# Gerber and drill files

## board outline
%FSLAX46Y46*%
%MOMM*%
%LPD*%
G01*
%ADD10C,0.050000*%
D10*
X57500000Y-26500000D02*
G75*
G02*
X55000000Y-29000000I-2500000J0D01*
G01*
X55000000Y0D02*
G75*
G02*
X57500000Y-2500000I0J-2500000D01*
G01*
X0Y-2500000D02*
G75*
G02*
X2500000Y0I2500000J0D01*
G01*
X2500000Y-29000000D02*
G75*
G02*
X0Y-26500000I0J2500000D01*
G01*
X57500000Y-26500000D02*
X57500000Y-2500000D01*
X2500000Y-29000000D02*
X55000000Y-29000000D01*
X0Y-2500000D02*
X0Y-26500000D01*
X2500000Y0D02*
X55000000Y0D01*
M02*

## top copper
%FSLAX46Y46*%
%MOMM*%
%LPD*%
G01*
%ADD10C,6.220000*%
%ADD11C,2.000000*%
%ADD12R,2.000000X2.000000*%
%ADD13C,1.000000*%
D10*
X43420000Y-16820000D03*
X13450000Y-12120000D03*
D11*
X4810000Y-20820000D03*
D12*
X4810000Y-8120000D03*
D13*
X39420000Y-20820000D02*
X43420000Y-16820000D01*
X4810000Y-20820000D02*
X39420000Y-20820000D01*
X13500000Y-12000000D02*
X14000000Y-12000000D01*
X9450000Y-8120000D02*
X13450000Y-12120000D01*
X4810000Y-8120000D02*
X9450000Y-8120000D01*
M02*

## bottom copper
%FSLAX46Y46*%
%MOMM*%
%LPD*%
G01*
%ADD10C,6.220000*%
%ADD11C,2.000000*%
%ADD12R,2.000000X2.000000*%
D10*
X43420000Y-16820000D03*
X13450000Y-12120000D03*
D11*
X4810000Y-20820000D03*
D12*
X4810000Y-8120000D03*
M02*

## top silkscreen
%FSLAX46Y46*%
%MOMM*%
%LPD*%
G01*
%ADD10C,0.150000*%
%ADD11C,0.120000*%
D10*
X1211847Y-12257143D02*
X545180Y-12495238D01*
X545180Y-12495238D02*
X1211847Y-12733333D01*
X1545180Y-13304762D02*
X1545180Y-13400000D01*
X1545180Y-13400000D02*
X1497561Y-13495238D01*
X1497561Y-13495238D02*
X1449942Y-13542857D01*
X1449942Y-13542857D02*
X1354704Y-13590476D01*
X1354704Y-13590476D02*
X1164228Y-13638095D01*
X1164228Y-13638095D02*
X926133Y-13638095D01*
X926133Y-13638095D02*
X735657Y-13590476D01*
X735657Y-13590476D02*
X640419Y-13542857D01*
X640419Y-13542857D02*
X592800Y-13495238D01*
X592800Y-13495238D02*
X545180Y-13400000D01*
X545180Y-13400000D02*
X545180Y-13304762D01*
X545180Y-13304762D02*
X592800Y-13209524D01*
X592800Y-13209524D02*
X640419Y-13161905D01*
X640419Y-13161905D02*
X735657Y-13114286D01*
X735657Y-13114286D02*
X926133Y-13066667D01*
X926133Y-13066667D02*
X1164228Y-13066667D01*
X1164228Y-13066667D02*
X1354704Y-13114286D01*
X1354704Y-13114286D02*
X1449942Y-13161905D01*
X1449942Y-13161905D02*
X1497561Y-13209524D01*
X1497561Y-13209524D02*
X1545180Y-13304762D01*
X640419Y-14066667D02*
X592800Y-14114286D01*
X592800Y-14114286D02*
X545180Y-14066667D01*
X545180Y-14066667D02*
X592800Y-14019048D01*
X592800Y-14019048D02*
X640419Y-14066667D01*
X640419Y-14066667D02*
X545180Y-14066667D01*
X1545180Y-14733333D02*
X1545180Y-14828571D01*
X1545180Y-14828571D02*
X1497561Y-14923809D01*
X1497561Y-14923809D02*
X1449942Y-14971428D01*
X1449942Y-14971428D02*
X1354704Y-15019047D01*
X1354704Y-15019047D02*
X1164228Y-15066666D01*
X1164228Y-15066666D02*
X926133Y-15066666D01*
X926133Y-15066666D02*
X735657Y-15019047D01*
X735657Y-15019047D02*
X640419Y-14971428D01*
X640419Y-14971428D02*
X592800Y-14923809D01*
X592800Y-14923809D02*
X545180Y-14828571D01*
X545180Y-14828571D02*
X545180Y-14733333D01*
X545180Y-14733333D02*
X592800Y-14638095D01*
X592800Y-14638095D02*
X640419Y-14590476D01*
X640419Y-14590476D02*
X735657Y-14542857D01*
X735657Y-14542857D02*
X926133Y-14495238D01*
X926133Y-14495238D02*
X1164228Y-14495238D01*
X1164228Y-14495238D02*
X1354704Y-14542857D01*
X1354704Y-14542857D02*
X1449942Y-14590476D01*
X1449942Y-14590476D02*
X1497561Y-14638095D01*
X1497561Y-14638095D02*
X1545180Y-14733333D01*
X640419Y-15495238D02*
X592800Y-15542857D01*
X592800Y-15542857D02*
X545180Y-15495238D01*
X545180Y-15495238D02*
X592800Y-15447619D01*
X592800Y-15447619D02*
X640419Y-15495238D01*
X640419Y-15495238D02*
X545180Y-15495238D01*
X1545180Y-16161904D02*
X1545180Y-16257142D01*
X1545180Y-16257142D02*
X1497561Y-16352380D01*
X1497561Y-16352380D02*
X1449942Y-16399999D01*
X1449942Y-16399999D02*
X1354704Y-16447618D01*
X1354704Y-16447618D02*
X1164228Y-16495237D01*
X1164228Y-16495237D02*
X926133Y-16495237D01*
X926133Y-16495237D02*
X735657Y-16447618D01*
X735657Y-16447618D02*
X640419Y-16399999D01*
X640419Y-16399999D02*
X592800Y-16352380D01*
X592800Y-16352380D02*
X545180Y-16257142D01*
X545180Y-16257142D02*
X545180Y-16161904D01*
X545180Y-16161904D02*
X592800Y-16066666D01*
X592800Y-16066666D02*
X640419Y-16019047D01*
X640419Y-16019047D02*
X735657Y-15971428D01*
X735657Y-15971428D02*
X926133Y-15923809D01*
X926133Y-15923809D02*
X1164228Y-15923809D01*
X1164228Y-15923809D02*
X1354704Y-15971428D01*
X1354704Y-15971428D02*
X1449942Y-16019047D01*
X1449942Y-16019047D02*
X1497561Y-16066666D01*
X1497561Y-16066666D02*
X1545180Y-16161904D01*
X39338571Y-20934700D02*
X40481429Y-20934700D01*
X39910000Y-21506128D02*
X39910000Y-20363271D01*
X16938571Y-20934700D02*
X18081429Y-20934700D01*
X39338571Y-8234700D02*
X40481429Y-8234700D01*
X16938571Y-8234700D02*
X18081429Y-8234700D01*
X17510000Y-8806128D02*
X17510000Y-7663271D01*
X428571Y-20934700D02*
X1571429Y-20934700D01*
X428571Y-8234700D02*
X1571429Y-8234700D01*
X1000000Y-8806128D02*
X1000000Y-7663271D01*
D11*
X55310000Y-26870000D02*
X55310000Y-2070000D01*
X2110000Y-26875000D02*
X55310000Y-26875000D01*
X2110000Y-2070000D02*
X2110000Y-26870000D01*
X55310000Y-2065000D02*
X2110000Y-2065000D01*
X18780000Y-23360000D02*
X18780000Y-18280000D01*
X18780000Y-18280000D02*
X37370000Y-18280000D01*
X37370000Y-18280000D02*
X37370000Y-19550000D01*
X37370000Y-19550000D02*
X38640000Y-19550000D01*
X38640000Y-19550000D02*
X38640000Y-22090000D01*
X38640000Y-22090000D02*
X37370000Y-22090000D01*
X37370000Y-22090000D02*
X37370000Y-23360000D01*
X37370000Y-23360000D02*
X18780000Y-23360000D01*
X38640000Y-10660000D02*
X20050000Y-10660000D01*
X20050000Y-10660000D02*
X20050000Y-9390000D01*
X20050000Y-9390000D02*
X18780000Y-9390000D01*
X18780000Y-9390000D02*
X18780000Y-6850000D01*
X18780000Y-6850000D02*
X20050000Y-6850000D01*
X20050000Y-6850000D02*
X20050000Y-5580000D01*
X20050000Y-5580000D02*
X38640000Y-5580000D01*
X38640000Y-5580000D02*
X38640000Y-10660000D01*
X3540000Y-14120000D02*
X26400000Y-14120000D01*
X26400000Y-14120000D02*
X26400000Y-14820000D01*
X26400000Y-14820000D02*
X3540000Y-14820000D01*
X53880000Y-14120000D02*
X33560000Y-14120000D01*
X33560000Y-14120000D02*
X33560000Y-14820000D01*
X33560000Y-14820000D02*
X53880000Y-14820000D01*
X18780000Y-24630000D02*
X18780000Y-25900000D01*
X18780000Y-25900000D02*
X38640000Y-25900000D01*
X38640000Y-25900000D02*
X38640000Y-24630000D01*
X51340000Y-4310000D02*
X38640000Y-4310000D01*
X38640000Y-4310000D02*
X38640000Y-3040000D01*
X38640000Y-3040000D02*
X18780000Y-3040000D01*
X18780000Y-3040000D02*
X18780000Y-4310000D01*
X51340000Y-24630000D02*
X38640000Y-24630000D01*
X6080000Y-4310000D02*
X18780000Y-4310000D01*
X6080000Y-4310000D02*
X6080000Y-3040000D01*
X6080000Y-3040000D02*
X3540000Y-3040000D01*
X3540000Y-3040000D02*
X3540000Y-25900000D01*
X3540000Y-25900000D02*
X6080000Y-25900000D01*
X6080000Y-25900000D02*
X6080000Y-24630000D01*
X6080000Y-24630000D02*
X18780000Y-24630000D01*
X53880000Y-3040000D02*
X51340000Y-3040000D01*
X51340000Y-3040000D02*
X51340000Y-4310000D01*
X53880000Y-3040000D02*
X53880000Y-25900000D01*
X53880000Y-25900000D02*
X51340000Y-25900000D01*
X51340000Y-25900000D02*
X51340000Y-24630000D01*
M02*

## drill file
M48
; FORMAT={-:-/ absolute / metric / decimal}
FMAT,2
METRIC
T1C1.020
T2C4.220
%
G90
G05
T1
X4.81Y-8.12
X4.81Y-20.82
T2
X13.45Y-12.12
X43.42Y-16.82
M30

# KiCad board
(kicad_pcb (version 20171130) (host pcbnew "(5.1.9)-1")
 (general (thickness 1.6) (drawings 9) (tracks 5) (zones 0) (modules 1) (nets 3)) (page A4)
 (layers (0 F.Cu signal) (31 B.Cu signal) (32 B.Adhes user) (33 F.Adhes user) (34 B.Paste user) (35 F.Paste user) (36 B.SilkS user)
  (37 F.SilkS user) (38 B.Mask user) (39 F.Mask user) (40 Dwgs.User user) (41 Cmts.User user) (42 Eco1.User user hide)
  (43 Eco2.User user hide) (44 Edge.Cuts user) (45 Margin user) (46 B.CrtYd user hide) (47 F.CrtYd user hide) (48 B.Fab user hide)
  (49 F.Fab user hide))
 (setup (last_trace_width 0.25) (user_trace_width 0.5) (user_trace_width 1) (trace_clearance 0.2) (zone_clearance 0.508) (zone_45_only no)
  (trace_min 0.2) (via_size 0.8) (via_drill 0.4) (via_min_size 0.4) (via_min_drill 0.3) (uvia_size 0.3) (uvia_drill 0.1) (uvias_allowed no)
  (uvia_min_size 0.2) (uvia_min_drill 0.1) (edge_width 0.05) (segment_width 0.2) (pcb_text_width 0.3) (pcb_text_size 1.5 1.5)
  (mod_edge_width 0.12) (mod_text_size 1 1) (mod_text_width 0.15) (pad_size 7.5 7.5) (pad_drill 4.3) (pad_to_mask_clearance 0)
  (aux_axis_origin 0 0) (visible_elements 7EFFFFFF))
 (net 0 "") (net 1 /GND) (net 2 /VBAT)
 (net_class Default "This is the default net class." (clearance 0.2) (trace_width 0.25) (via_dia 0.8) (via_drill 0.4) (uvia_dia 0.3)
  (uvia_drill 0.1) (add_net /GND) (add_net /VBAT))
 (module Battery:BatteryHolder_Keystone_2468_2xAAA (layer F.Cu) (at 4.81 8.12)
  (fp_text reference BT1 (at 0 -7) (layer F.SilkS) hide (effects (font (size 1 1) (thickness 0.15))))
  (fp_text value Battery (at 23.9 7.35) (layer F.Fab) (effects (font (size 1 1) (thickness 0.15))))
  (fp_line (start 50.5 18.75) (end 50.5 -6.05) (layer F.SilkS) (width 0.12))
  (fp_line (start -2.7 18.755) (end 50.5 18.755) (layer F.SilkS) (width 0.12))
  (fp_line (start -2.7 -6.05) (end -2.7 18.75) (layer F.SilkS) (width 0.12))
  (fp_line (start 50.5 -6.055) (end -2.7 -6.055) (layer F.SilkS) (width 0.12))
  (fp_line (start 13.97 15.24) (end 13.97 10.16) (layer F.SilkS) (width 0.12))
  (fp_line (start 13.97 10.16) (end 32.56 10.16) (layer F.SilkS) (width 0.12))
  (fp_line (start 32.56 10.16) (end 32.56 11.43) (layer F.SilkS) (width 0.12))
  (fp_line (start 32.56 11.43) (end 33.83 11.43) (layer F.SilkS) (width 0.12))
  (fp_line (start 33.83 11.43) (end 33.83 13.97) (layer F.SilkS) (width 0.12))
  (fp_line (start 33.83 13.97) (end 32.56 13.97) (layer F.SilkS) (width 0.12))
  (fp_line (start 32.56 13.97) (end 32.56 15.24) (layer F.SilkS) (width 0.12))
  (fp_line (start 32.56 15.24) (end 13.97 15.24) (layer F.SilkS) (width 0.12))
  (fp_line (start 33.83 2.54) (end 15.24 2.54) (layer F.SilkS) (width 0.12))
  (fp_line (start 15.24 2.54) (end 15.24 1.27) (layer F.SilkS) (width 0.12))
  (fp_line (start 15.24 1.27) (end 13.97 1.27) (layer F.SilkS) (width 0.12))
  (fp_line (start 13.97 1.27) (end 13.97 -1.27) (layer F.SilkS) (width 0.12))
  (fp_line (start 13.97 -1.27) (end 15.24 -1.27) (layer F.SilkS) (width 0.12))
  (fp_line (start 15.24 -1.27) (end 15.24 -2.54) (layer F.SilkS) (width 0.12))
  (fp_line (start 15.24 -2.54) (end 33.83 -2.54) (layer F.SilkS) (width 0.12))
  (fp_line (start 33.83 -2.54) (end 33.83 2.54) (layer F.SilkS) (width 0.12))
  (fp_line (start -1.27 6) (end 21.59 6) (layer F.SilkS) (width 0.12))
  (fp_line (start 21.59 6) (end 21.59 6.7) (layer F.SilkS) (width 0.12))
  (fp_line (start 21.59 6.7) (end -1.27 6.7) (layer F.SilkS) (width 0.12))
  (fp_line (start 49.07 6) (end 28.75 6) (layer F.SilkS) (width 0.12))
  (fp_line (start 28.75 6) (end 28.75 6.7) (layer F.SilkS) (width 0.12))
  (fp_line (start 28.75 6.7) (end 49.07 6.7) (layer F.SilkS) (width 0.12))
  (fp_line (start 13.97 16.51) (end 13.97 17.78) (layer F.SilkS) (width 0.12))
  (fp_line (start 13.97 17.78) (end 33.83 17.78) (layer F.SilkS) (width 0.12))
  (fp_line (start 33.83 17.78) (end 33.83 16.51) (layer F.SilkS) (width 0.12))
  (fp_line (start 46.53 -3.81) (end 33.83 -3.81) (layer F.SilkS) (width 0.12))
  (fp_line (start 33.83 -3.81) (end 33.83 -5.08) (layer F.SilkS) (width 0.12))
  (fp_line (start 33.83 -5.08) (end 13.97 -5.08) (layer F.SilkS) (width 0.12))
  (fp_line (start 13.97 -5.08) (end 13.97 -3.81) (layer F.SilkS) (width 0.12))
  (fp_line (start 46.53 16.51) (end 33.83 16.51) (layer F.SilkS) (width 0.12))
  (fp_line (start 1.27 -3.81) (end 13.97 -3.81) (layer F.SilkS) (width 0.12))
  (fp_line (start 1.27 -3.81) (end 1.27 -5.08) (layer F.SilkS) (width 0.12))
  (fp_line (start 1.27 -5.08) (end -1.27 -5.08) (layer F.SilkS) (width 0.12))
  (fp_line (start -1.27 -5.08) (end -1.27 17.78) (layer F.SilkS) (width 0.12))
  (fp_line (start -1.27 17.78) (end 1.27 17.78) (layer F.SilkS) (width 0.12))
  (fp_line (start 1.27 17.78) (end 1.27 16.51) (layer F.SilkS) (width 0.12))
  (fp_line (start 1.27 16.51) (end 13.97 16.51) (layer F.SilkS) (width 0.12))
  (fp_line (start 49.07 -5.08) (end 46.53 -5.08) (layer F.SilkS) (width 0.12))
  (fp_line (start 46.53 -5.08) (end 46.53 -3.81) (layer F.SilkS) (width 0.12))
  (fp_line (start 49.07 -5.08) (end 49.07 17.78) (layer F.SilkS) (width 0.12))
  (fp_line (start 49.07 17.78) (end 46.53 17.78) (layer F.SilkS) (width 0.12))
  (fp_line (start 46.53 17.78) (end 46.53 16.51) (layer F.SilkS) (width 0.12))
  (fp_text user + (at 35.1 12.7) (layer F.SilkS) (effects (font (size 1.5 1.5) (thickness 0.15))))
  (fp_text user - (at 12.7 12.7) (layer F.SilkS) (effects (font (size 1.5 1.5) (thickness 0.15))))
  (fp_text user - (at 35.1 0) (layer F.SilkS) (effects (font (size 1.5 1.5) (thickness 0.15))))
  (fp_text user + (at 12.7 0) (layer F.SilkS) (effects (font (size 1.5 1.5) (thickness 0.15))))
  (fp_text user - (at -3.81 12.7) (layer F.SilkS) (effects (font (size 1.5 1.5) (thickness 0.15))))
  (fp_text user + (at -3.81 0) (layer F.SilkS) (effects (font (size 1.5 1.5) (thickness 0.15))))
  (pad 2 thru_hole circle (at 38.61 8.7) (size 6.22 6.22) (drill 4.22) (layers *.Cu *.Mask) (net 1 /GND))
  (pad 1 thru_hole circle (at 8.64 4) (size 6.22 6.22) (drill 4.22) (layers *.Cu *.Mask) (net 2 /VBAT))
  (pad 2 thru_hole circle (at 0 12.7) (size 2 2) (drill 1.02) (layers *.Cu *.Mask) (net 1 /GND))
  (pad 1 thru_hole rect (at 0 0) (size 2 2) (drill 1.02) (layers *.Cu *.Mask) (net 2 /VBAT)))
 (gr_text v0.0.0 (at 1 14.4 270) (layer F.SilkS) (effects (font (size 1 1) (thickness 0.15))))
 (gr_arc (start 55 26.5) (end 55 29) (angle -90) (layer Edge.Cuts) (width 0.05))
 (gr_arc (start 55 2.5) (end 57.5 2.5) (angle -90) (layer Edge.Cuts) (width 0.05))
 (gr_arc (start 2.5 2.5) (end 2.5 0) (angle -90) (layer Edge.Cuts) (width 0.05))
 (gr_arc (start 2.5 26.5) (end 0 26.5) (angle -90) (layer Edge.Cuts) (width 0.05))
 (gr_line (start 57.5 26.5) (end 57.5 2.5) (layer Edge.Cuts) (width 0.05))
 (gr_line (start 2.5 29) (end 55 29) (layer Edge.Cuts) (width 0.05))
 (gr_line (start 0 2.5) (end 0 26.5) (layer Edge.Cuts) (width 0.05))
 (gr_line (start 2.5 0) (end 55 0) (layer Edge.Cuts) (width 0.05))
 (segment (start 39.42 20.82) (end 43.42 16.82) (width 1) (layer F.Cu) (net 1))
 (segment (start 4.81 20.82) (end 39.42 20.82) (width 1) (layer F.Cu) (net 1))
 (segment (start 13.5 12) (end 14 12) (width 1) (layer F.Cu) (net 2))
 (segment (start 9.45 8.12) (end 13.45 12.12) (width 1) (layer F.Cu) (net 2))
 (segment (start 4.81 8.12) (end 9.45 8.12) (width 1) (layer F.Cu) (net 2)))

